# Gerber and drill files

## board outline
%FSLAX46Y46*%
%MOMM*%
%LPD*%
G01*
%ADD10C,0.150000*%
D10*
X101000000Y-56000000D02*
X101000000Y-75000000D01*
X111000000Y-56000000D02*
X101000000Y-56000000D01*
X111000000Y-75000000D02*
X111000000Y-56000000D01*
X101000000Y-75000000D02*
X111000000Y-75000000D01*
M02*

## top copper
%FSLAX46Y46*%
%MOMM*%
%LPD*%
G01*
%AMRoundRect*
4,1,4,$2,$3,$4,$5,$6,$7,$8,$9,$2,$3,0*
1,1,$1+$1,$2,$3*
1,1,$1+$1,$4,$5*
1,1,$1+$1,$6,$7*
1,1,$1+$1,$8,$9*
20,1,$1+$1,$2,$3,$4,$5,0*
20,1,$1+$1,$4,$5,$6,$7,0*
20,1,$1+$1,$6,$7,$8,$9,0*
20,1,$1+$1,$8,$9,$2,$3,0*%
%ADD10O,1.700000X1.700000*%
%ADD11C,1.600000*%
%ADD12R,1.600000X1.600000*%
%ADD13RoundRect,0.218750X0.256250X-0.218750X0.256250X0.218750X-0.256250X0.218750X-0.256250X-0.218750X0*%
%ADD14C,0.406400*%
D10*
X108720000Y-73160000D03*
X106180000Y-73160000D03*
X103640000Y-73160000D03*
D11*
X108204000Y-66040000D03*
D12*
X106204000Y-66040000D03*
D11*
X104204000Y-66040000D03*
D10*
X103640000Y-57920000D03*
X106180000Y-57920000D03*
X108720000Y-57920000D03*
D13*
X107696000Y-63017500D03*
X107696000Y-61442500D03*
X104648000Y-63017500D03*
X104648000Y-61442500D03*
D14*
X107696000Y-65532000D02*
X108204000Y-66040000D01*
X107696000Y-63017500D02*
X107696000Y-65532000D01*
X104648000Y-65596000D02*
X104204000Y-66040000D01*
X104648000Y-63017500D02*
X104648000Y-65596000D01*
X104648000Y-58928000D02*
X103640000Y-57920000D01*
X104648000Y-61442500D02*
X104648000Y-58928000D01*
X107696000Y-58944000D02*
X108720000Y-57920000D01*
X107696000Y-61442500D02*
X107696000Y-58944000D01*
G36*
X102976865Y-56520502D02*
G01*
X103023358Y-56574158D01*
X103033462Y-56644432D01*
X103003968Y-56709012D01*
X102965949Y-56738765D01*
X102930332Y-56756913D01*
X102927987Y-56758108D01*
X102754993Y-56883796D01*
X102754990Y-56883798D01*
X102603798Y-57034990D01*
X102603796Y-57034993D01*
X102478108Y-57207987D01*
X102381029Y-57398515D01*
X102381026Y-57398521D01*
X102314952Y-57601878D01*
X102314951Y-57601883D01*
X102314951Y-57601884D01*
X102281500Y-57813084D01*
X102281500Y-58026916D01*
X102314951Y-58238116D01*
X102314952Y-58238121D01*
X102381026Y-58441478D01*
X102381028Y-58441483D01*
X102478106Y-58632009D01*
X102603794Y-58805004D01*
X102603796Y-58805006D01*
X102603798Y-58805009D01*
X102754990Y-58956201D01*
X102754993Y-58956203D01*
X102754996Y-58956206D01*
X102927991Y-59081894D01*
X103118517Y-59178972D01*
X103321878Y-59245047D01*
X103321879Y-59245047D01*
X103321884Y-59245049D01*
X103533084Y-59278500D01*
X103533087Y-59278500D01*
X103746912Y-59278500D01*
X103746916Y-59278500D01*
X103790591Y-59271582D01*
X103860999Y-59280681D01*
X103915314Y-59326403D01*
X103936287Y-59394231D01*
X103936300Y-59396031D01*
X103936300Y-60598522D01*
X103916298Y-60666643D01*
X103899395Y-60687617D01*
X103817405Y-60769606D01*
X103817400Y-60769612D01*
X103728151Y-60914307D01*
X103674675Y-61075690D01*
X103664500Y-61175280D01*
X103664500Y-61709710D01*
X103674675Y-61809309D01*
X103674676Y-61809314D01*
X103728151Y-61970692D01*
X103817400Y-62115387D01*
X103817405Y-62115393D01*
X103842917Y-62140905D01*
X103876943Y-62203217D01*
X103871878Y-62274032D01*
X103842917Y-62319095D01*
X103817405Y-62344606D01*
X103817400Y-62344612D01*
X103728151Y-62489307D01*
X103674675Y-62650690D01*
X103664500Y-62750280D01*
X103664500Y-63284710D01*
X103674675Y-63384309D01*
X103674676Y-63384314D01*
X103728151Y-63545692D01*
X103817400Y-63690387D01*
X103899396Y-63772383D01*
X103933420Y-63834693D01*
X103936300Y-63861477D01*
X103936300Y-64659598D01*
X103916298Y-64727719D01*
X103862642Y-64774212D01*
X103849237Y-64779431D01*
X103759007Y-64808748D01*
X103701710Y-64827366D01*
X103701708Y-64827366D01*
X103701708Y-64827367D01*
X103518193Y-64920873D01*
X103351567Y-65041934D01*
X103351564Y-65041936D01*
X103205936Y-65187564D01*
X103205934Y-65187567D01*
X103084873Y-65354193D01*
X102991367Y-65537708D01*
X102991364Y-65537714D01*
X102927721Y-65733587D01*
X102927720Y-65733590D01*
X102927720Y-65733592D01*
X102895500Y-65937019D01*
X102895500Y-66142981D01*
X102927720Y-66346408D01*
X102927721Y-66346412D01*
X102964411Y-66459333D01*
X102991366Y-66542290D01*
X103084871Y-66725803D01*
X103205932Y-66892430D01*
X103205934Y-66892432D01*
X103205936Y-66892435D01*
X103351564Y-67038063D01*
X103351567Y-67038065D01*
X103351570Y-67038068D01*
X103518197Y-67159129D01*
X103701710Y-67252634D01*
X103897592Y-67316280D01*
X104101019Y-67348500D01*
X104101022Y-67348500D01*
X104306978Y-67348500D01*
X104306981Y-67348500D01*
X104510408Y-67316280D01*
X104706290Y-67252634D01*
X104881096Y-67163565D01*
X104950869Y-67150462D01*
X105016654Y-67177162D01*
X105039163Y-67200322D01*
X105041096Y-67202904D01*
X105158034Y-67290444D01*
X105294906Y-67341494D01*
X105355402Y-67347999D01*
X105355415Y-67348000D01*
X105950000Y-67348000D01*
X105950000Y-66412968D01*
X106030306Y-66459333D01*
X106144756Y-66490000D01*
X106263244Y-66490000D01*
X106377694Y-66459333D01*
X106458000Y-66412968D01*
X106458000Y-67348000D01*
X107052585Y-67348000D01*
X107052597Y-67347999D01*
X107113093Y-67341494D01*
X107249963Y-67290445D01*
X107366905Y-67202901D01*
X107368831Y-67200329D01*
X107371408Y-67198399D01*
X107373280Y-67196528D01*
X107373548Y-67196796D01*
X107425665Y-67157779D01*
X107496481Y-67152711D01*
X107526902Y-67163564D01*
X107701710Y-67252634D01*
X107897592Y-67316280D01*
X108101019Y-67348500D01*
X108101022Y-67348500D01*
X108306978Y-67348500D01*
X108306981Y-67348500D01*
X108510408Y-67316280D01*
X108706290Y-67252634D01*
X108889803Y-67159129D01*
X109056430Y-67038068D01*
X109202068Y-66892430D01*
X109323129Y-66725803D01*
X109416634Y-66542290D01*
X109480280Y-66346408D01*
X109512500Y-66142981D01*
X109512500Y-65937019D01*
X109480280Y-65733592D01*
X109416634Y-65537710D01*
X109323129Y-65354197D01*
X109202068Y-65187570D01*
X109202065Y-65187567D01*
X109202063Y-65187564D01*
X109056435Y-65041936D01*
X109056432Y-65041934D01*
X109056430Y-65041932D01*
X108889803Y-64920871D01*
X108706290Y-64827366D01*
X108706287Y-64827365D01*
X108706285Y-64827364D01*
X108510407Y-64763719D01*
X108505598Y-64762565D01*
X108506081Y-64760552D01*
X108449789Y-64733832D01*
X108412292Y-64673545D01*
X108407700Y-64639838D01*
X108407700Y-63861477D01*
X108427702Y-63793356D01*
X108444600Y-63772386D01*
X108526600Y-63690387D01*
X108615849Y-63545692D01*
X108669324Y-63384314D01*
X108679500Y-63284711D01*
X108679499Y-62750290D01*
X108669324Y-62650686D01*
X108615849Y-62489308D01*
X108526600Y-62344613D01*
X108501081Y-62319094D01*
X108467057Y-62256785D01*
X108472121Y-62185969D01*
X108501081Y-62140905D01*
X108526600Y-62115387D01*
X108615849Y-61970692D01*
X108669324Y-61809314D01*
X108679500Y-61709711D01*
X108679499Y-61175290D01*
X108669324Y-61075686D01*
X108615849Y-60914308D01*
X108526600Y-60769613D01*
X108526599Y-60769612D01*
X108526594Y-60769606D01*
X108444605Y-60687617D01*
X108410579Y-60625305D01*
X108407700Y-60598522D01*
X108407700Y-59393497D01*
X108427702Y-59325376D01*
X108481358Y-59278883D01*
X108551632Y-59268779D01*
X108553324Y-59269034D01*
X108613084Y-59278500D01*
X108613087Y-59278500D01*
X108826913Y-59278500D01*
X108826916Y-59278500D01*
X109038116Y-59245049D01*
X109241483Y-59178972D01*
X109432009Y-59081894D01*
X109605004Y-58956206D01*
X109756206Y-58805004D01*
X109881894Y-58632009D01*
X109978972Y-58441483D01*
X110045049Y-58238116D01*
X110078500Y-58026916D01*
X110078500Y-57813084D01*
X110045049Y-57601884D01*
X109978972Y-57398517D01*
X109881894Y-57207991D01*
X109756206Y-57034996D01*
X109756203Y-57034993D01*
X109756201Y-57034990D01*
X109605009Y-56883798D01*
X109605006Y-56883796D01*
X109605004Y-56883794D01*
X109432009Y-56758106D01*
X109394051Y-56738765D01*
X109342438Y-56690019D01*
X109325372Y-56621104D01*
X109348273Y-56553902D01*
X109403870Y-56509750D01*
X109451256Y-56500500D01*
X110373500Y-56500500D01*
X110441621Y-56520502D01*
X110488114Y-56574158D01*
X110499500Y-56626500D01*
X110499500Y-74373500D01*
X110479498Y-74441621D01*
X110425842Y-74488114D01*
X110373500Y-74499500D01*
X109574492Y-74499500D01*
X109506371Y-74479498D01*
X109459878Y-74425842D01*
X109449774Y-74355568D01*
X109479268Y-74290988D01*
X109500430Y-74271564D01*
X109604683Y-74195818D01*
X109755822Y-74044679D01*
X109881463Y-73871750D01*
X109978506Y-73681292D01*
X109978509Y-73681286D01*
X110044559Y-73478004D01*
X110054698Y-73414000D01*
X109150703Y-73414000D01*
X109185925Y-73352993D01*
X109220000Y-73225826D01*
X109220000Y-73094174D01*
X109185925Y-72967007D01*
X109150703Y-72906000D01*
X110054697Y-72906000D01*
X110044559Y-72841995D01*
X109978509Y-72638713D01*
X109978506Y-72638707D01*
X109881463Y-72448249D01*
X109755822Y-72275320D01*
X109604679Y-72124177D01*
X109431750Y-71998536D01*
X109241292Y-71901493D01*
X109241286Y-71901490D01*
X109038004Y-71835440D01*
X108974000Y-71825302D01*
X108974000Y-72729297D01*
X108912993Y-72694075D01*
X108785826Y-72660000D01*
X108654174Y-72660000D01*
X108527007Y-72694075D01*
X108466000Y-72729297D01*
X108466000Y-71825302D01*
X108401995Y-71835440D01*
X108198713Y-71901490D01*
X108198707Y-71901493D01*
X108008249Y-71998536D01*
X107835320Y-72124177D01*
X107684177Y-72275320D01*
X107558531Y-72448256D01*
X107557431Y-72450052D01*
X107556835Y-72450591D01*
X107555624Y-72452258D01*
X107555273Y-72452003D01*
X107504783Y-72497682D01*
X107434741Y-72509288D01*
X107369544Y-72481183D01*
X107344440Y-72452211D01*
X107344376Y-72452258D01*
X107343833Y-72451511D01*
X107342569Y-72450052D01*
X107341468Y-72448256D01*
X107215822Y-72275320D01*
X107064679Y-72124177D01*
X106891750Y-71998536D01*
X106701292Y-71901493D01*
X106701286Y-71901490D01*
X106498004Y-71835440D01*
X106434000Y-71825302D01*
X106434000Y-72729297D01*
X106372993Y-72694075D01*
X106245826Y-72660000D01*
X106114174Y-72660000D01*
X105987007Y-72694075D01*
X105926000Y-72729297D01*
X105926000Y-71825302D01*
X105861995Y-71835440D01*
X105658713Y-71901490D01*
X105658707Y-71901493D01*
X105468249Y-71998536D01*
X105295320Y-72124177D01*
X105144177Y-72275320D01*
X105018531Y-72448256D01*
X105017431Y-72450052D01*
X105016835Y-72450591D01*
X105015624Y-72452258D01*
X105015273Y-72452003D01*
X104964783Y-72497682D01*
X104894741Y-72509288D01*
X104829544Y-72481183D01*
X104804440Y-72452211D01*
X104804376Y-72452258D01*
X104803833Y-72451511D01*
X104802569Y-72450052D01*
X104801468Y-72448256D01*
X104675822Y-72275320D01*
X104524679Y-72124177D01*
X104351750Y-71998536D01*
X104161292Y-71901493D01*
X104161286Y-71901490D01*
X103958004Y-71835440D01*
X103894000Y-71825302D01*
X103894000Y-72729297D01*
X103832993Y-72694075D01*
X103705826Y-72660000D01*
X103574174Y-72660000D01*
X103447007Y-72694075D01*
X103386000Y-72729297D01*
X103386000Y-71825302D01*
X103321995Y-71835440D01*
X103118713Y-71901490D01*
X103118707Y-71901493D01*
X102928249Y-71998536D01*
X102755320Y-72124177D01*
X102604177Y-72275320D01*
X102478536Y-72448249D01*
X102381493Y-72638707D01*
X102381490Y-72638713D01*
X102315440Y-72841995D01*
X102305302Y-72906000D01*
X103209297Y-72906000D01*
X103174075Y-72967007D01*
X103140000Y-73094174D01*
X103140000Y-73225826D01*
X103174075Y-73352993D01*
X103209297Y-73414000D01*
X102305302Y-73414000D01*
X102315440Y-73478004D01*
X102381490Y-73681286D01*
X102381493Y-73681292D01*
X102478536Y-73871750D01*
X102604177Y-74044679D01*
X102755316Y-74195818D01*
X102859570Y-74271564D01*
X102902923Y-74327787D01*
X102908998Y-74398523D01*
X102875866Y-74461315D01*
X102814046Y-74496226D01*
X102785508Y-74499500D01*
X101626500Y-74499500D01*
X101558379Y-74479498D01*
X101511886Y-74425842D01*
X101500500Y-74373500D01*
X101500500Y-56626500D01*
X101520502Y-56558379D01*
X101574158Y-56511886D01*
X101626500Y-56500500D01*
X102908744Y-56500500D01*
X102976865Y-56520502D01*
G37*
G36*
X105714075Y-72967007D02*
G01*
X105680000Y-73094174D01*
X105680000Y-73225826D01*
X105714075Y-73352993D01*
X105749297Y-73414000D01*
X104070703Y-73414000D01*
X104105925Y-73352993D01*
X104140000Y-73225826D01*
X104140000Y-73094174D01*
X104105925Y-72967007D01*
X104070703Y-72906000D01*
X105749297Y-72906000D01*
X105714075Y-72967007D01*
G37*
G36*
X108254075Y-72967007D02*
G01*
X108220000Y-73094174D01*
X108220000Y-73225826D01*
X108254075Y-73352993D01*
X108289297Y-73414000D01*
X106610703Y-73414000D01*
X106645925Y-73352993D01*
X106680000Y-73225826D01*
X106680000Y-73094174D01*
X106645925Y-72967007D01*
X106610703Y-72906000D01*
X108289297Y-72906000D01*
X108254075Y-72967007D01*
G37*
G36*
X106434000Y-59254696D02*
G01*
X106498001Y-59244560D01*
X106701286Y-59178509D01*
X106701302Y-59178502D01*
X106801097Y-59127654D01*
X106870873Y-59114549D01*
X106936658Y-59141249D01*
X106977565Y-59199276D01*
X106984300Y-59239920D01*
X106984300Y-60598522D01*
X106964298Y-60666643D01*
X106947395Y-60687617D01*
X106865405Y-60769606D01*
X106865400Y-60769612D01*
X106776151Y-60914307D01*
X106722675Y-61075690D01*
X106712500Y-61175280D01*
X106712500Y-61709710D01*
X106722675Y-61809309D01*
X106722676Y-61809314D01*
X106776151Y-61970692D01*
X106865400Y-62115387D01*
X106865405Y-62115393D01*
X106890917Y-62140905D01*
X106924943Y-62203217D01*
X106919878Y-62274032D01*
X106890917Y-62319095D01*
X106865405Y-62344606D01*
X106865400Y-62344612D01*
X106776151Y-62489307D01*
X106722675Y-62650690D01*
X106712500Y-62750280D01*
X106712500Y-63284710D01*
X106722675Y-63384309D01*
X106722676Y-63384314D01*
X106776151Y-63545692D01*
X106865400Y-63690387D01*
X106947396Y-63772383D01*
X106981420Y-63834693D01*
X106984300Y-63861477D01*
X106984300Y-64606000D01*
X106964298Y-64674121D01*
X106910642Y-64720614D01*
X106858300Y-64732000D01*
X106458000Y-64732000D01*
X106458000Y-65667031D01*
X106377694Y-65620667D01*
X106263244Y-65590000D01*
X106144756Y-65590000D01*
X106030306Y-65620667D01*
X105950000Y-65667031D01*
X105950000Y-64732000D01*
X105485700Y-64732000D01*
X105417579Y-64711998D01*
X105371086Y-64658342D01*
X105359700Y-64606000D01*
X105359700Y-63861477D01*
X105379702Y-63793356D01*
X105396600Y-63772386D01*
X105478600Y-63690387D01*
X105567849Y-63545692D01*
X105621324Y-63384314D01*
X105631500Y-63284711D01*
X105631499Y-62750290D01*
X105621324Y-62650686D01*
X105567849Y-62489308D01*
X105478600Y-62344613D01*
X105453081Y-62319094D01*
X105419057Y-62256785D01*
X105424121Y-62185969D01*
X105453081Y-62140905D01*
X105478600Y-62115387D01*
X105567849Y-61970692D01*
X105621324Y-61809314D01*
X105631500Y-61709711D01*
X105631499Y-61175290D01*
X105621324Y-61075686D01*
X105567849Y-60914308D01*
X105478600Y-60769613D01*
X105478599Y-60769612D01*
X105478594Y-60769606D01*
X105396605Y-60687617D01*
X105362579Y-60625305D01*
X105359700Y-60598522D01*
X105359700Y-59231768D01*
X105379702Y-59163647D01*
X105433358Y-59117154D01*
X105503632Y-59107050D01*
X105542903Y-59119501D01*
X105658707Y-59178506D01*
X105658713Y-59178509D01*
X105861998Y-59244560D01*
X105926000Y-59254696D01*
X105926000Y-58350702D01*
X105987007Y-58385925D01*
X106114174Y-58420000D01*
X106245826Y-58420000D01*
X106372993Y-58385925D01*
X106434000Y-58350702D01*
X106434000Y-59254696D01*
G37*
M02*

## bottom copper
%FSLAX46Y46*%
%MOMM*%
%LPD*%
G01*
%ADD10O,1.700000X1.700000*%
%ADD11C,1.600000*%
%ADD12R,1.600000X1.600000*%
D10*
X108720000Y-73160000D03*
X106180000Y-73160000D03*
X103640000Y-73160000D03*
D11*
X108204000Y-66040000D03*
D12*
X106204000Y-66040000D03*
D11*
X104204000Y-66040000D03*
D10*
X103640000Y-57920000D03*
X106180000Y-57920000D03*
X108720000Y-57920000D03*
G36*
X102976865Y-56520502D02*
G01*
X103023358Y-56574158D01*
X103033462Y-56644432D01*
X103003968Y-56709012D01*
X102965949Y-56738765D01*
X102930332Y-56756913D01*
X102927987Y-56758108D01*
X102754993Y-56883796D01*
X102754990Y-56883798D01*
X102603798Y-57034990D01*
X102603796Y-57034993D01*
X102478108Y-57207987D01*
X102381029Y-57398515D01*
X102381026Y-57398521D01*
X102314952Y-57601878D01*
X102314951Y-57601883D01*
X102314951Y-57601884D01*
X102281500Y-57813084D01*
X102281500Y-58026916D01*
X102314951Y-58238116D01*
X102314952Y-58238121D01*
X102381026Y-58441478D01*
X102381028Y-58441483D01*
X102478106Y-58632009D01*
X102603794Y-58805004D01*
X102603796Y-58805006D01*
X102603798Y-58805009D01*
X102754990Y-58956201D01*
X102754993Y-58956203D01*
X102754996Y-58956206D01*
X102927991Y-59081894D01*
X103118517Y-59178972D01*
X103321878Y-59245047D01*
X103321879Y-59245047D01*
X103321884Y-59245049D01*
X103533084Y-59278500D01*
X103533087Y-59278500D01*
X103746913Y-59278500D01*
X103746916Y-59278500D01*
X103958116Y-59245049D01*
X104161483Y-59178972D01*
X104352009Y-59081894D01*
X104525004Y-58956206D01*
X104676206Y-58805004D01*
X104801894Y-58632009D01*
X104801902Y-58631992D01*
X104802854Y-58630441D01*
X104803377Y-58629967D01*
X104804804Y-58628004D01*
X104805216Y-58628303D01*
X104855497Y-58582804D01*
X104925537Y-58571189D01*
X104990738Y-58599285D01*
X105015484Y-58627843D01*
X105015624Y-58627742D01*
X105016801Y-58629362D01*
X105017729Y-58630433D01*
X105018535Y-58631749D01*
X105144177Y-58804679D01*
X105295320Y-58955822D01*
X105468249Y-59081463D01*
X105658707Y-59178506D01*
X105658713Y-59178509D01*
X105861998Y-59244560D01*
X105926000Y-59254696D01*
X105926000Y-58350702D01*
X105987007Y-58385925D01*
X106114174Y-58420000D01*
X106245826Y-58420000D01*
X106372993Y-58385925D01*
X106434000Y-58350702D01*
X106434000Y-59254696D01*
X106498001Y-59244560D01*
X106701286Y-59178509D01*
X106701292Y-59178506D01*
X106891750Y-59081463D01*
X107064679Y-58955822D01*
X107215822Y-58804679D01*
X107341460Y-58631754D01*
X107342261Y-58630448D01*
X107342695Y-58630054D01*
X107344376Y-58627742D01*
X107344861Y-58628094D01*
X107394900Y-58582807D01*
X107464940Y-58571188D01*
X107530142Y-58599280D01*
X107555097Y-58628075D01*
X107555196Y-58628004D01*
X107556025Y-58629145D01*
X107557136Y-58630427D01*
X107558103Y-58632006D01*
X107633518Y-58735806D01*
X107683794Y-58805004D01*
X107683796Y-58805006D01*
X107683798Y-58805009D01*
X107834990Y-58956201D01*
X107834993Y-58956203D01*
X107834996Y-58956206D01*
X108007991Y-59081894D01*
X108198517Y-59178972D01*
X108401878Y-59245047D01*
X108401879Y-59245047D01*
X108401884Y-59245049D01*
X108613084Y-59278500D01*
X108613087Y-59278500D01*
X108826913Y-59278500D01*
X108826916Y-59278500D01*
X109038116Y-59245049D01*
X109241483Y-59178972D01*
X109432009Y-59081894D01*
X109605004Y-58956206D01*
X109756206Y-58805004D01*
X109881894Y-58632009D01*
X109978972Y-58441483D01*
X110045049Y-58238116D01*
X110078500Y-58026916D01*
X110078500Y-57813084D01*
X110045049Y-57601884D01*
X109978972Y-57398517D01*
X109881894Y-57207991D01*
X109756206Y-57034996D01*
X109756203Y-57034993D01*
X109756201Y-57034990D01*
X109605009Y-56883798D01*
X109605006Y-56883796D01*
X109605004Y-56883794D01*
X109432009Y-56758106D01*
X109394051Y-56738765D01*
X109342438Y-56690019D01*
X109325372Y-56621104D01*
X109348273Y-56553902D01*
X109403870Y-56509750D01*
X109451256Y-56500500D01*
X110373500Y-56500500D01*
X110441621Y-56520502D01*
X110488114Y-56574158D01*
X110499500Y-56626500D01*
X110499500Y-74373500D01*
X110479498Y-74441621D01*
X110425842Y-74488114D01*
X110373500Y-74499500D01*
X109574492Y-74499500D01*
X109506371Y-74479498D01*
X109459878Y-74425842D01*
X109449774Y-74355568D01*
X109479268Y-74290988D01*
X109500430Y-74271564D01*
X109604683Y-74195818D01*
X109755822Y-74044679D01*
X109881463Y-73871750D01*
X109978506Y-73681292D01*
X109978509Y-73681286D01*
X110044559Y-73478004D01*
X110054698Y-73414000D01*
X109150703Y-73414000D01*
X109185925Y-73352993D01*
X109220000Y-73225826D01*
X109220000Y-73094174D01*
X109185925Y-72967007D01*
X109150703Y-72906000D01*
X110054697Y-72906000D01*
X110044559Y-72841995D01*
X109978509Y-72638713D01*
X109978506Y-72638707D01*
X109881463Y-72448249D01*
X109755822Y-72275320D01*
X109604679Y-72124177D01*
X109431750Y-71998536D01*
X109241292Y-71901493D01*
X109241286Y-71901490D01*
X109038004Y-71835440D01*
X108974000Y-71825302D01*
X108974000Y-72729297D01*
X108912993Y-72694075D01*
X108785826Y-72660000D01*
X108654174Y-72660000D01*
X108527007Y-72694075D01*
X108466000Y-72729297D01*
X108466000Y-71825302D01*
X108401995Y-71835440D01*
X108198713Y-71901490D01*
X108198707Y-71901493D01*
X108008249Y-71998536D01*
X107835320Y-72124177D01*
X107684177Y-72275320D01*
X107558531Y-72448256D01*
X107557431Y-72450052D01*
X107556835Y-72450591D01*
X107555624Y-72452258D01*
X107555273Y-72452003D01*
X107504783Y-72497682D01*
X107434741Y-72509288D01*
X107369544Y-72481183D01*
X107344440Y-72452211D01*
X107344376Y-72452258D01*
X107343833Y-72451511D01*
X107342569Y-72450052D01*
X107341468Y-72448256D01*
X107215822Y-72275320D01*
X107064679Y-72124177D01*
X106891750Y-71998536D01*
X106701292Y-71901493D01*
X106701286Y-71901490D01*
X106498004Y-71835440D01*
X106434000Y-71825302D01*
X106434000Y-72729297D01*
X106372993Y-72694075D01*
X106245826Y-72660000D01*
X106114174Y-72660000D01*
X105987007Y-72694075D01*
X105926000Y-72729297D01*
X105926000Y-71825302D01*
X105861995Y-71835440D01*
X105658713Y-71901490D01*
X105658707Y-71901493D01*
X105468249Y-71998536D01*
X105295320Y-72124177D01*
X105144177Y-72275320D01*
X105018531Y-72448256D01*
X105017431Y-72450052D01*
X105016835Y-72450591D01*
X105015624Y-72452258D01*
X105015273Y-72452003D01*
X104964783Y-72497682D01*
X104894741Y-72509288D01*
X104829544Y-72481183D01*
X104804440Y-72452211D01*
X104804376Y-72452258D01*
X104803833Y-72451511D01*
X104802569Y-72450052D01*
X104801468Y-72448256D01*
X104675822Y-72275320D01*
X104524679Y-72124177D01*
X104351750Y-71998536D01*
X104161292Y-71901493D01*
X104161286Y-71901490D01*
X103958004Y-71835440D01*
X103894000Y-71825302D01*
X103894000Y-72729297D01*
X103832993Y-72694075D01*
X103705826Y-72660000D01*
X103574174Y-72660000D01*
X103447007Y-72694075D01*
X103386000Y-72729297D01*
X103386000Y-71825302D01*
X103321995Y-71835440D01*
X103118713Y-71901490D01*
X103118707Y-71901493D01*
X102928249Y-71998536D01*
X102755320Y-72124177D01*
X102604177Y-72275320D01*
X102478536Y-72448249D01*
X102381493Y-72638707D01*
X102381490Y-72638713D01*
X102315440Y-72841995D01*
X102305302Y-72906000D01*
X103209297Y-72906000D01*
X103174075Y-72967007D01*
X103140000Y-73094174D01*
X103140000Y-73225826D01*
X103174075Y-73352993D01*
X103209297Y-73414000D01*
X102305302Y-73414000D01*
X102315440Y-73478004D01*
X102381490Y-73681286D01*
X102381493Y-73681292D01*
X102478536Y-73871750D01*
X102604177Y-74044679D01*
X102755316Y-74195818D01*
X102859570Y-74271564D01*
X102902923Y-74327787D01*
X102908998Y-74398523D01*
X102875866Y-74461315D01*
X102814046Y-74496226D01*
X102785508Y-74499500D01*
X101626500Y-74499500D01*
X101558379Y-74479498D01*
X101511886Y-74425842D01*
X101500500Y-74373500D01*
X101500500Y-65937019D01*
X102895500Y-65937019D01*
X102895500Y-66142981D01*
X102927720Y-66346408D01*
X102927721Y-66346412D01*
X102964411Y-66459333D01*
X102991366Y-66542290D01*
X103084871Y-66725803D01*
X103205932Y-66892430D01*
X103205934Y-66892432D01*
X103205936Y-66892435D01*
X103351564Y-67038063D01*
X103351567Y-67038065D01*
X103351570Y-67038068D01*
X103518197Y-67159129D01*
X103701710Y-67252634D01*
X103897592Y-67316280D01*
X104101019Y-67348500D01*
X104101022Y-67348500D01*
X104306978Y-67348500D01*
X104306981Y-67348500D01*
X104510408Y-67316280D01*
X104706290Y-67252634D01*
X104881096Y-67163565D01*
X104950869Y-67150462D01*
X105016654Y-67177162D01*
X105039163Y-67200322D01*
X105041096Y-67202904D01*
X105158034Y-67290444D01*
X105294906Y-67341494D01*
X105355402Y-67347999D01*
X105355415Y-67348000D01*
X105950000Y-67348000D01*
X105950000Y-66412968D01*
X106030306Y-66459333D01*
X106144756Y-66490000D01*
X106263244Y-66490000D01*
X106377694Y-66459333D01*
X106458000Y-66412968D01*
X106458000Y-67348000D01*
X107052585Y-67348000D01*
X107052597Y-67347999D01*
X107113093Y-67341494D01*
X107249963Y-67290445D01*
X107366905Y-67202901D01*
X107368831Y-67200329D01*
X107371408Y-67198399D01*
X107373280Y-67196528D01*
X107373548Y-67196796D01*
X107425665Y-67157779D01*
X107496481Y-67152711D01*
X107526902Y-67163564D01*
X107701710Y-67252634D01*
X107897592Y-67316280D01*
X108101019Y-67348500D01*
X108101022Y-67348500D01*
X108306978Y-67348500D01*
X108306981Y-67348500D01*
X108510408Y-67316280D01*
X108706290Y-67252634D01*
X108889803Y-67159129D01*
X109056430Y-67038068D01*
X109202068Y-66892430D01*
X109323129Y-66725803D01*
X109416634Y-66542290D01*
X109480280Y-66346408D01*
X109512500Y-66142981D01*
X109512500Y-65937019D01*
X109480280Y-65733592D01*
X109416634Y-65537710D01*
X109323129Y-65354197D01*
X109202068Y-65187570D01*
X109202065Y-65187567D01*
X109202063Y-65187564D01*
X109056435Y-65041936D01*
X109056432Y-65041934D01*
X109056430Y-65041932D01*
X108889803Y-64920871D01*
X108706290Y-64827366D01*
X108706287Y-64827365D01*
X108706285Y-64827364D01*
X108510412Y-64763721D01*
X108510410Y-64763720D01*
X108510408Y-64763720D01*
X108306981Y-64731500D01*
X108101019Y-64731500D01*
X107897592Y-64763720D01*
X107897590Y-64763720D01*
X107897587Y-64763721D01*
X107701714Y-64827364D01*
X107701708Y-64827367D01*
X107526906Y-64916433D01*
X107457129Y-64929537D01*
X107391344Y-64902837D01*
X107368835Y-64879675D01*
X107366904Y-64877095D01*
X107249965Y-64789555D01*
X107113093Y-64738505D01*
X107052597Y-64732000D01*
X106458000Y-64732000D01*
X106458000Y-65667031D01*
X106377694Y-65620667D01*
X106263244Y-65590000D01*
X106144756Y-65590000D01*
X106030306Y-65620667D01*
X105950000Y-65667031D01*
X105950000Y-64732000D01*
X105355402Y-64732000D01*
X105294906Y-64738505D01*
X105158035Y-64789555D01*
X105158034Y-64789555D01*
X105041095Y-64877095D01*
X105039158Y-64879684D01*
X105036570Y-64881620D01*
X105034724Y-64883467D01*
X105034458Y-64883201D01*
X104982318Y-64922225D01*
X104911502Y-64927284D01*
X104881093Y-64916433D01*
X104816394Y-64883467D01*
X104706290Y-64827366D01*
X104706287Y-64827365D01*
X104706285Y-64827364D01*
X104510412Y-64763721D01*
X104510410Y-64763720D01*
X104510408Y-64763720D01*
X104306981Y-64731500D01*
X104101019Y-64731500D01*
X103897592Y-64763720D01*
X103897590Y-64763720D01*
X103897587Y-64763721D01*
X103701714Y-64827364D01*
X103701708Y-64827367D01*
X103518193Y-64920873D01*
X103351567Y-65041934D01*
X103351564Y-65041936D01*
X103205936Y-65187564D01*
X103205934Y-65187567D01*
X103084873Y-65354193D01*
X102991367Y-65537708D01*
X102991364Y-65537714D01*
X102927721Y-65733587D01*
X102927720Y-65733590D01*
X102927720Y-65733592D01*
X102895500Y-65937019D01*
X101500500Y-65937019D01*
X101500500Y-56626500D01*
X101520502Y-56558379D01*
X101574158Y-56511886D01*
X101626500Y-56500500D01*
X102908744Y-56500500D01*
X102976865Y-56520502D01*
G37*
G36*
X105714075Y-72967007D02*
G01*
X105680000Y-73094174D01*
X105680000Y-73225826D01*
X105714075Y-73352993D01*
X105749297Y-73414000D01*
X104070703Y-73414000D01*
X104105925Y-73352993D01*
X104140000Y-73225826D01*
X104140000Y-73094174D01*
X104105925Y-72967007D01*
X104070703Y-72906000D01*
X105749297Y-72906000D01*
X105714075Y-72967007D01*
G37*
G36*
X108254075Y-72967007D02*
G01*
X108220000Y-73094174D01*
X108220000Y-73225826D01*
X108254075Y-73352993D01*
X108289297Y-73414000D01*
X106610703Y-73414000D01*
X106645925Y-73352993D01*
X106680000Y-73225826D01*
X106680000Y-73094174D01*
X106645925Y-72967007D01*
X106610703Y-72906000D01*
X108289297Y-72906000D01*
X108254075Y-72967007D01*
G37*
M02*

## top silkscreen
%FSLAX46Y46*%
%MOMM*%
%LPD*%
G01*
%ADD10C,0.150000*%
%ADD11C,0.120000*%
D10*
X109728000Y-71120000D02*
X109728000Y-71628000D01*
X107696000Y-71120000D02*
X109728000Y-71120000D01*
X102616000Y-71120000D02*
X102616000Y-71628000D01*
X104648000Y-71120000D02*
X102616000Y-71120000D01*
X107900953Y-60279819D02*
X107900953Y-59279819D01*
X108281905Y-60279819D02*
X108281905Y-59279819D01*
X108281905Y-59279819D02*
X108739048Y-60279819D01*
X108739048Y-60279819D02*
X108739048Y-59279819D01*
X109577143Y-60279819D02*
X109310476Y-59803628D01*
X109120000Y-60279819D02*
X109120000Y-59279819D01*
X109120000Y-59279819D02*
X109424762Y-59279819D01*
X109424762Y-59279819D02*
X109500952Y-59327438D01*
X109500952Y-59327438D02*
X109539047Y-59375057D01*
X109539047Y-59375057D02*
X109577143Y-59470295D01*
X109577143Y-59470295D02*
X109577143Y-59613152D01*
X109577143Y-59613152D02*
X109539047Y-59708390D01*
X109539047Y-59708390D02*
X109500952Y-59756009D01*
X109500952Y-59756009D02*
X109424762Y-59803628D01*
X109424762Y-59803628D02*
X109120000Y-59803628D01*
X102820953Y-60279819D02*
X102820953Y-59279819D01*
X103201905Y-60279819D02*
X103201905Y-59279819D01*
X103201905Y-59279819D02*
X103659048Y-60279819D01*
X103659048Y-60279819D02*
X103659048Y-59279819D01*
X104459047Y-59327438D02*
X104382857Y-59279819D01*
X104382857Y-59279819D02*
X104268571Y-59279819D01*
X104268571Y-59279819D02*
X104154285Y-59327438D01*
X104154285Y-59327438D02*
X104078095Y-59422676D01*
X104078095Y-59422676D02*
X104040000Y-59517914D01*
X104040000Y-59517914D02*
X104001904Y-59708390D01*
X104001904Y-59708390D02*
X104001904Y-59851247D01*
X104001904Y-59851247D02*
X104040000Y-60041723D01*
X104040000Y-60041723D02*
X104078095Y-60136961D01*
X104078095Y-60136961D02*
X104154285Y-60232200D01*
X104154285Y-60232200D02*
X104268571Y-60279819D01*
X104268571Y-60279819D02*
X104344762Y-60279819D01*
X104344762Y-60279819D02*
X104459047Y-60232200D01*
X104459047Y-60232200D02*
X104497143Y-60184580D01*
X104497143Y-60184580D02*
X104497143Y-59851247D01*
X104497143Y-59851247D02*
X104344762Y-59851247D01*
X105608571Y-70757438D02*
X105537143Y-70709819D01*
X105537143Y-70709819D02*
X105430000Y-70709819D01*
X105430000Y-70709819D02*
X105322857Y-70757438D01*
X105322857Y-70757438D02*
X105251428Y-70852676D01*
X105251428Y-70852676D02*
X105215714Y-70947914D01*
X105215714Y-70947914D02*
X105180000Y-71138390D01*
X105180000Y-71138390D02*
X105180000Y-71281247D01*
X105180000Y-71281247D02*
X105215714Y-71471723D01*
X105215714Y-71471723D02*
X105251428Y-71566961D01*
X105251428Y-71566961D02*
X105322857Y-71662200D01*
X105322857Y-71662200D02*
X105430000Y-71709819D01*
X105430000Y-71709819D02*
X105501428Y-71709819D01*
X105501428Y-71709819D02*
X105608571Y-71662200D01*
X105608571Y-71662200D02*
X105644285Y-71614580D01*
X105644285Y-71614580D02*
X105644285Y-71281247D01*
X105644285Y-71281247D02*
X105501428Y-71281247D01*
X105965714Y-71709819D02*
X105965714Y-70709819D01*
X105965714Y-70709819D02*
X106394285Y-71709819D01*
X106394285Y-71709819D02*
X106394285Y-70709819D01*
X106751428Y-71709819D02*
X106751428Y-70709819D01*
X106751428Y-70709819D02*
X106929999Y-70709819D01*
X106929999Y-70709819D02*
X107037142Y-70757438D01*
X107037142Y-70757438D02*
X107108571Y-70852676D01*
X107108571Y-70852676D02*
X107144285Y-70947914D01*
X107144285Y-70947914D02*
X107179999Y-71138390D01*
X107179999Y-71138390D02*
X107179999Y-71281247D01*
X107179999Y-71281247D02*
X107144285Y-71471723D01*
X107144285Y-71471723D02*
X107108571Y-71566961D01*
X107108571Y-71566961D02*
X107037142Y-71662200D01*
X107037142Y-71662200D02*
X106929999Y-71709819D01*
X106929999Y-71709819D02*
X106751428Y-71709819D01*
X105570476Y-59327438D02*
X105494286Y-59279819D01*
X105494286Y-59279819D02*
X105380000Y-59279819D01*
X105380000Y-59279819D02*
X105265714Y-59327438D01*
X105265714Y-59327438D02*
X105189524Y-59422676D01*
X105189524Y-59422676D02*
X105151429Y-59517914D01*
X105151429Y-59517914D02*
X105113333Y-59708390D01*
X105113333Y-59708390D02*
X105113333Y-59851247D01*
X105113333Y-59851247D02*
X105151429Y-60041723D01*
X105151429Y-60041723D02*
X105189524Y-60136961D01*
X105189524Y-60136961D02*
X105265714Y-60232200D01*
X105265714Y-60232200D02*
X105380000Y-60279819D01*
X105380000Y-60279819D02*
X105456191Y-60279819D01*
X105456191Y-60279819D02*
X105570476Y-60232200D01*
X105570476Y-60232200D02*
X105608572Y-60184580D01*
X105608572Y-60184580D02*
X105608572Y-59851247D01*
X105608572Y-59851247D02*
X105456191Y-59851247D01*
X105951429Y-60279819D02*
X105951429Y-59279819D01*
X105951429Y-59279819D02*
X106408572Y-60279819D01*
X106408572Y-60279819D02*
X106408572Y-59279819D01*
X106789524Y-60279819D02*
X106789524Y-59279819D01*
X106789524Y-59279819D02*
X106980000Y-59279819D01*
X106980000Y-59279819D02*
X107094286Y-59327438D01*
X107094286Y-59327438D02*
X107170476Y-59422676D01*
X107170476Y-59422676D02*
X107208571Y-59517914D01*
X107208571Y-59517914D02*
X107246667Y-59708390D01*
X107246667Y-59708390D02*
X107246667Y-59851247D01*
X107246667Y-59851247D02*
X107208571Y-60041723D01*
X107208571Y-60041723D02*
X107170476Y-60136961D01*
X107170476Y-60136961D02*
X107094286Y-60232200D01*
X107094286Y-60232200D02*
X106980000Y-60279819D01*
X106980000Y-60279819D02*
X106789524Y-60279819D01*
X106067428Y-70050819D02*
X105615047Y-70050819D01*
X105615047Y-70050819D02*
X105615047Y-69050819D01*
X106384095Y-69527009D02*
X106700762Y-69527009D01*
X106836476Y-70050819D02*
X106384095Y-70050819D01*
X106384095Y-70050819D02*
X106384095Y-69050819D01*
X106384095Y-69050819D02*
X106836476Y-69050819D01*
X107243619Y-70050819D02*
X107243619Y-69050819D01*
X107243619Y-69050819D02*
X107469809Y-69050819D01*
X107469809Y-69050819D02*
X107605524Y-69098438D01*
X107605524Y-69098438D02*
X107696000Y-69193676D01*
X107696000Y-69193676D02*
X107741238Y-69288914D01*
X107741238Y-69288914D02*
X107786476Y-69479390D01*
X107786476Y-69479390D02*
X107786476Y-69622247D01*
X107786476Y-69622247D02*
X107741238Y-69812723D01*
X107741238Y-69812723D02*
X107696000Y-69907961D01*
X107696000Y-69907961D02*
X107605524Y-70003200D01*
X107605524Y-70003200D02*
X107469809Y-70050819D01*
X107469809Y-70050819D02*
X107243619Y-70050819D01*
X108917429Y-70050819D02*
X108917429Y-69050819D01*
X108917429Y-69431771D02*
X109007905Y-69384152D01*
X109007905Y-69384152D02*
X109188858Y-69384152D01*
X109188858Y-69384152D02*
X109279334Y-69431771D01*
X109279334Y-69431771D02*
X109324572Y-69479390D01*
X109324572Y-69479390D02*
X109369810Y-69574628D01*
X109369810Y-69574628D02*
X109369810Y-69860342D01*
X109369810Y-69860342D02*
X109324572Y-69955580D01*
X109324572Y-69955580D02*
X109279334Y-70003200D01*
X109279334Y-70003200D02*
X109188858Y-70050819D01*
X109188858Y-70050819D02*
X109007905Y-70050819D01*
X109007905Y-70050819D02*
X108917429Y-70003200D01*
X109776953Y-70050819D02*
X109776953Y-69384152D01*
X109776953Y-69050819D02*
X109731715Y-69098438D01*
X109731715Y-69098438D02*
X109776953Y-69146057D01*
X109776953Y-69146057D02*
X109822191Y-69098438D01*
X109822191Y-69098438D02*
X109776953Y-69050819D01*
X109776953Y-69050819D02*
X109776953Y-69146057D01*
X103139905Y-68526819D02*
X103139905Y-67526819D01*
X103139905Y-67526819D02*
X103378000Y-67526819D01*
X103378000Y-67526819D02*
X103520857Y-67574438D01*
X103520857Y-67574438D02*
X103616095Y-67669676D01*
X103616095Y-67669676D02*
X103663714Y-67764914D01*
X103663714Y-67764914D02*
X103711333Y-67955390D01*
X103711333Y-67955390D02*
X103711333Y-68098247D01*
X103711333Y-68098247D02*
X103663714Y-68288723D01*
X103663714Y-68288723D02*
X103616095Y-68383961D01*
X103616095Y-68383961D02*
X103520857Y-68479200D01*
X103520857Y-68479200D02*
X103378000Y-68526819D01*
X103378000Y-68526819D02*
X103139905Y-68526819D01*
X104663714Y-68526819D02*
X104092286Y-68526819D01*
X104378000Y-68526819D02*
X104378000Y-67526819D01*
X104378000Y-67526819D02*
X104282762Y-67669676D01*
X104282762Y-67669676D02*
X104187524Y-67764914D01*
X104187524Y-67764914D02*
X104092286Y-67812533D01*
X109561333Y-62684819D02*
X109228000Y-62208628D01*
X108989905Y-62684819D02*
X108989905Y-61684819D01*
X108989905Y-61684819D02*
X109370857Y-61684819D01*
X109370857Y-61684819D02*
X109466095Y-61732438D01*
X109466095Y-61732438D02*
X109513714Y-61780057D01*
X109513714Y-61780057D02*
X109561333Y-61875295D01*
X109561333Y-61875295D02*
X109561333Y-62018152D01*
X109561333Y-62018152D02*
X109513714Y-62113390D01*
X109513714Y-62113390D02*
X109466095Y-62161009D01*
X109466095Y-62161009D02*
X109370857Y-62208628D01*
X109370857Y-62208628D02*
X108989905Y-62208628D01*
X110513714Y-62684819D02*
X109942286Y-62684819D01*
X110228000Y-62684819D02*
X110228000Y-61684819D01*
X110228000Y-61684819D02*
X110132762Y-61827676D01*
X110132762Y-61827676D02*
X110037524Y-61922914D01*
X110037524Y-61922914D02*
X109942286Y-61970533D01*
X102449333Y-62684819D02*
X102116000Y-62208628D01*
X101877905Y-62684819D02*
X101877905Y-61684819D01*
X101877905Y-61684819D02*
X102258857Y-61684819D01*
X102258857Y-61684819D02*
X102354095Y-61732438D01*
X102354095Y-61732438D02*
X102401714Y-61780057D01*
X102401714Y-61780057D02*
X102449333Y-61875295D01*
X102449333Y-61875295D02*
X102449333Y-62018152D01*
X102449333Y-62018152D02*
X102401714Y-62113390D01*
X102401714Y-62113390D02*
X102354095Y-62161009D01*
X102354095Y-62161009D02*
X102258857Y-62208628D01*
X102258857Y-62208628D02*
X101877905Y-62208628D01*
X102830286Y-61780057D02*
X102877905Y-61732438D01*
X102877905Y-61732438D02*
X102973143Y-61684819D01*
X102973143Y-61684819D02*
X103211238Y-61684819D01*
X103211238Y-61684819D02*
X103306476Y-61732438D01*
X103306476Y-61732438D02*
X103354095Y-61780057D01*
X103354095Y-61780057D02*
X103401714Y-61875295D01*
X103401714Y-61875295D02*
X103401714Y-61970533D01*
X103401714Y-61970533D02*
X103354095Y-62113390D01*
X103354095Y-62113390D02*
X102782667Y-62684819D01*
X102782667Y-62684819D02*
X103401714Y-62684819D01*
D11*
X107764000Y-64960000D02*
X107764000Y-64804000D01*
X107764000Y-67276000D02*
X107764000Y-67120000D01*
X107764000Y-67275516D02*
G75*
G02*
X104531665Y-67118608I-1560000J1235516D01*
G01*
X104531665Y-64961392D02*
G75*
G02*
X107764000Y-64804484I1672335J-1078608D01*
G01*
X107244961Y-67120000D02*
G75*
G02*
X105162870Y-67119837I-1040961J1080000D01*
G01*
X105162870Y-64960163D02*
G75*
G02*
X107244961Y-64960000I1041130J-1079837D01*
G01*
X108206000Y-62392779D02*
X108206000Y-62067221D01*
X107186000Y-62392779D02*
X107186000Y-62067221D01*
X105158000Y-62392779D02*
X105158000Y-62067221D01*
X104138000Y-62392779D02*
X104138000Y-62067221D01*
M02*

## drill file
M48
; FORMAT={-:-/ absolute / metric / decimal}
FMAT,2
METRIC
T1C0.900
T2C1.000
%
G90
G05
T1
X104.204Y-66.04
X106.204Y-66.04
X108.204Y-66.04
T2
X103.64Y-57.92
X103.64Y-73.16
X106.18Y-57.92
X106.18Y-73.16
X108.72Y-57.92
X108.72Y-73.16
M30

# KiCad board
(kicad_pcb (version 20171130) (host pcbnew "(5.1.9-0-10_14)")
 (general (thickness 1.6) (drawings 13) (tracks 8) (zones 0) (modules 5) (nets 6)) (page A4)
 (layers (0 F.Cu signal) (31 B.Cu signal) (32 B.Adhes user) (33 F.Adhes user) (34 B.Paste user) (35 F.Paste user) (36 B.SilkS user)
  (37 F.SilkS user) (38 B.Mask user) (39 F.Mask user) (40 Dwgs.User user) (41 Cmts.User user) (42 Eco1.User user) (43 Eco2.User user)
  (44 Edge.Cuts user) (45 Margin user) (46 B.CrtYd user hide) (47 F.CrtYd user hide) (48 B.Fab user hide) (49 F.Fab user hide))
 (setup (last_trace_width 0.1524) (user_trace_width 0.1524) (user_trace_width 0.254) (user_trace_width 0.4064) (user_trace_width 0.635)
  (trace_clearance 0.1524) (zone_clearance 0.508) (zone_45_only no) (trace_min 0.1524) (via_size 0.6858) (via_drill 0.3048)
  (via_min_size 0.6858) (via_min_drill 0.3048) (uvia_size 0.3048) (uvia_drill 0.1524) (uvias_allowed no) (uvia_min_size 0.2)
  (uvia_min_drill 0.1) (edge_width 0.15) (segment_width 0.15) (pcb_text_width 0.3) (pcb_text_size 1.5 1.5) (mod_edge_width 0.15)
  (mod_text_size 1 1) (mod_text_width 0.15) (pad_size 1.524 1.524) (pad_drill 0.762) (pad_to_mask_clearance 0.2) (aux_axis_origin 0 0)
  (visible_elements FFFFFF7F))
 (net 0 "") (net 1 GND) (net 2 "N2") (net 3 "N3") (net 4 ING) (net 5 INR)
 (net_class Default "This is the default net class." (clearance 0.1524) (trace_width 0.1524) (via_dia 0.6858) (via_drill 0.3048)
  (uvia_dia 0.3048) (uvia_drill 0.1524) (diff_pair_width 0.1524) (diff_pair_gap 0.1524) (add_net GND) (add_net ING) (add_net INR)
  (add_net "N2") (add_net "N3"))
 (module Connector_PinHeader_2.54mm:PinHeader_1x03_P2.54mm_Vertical (layer B.Cu) (at 103.64 73.16 270)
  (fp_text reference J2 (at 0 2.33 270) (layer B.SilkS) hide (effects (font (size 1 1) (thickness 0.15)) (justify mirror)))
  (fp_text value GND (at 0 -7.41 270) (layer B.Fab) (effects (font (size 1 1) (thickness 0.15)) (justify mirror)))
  (pad 3 thru_hole oval (at 0 -5.08 270) (size 1.7 1.7) (drill 1) (layers *.Cu *.Mask) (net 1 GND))
  (pad 2 thru_hole oval (at 0 -2.54 270) (size 1.7 1.7) (drill 1) (layers *.Cu *.Mask) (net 1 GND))
  (pad 1 thru_hole oval (at 0 0 270) (size 1.7 1.7) (drill 1) (layers *.Cu *.Mask) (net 1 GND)))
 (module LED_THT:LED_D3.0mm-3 (layer F.Cu) (at 108.704 66.04 180)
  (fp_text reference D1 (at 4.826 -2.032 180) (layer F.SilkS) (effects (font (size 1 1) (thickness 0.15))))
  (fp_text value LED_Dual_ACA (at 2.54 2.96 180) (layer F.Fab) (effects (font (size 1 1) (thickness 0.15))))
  (fp_line (start 0.94 1.08) (end 0.94 1.236) (layer F.SilkS) (width 0.12))
  (fp_line (start 0.94 -1.236) (end 0.94 -1.08) (layer F.SilkS) (width 0.12))
  (fp_arc (start 2.5 0) (end 0.94 -1.235516) (angle 108.8) (layer F.SilkS) (width 0.12))
  (fp_arc (start 2.5 0) (end 0.94 1.235516) (angle -108.8) (layer F.SilkS) (width 0.12))
  (fp_arc (start 2.5 0) (end 1.459039 -1.08) (angle 87.9) (layer F.SilkS) (width 0.12))
  (fp_arc (start 2.5 0) (end 1.459039 1.08) (angle -87.9) (layer F.SilkS) (width 0.12))
  (pad 1 thru_hole circle (at 0.5 0 180) (size 1.6 1.6) (drill 0.9) (layers *.Cu *.Mask) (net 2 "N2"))
  (pad 2 thru_hole rect (at 2.5 0 180) (size 1.6 1.6) (drill 0.9) (layers *.Cu *.Mask) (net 1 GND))
  (pad 3 thru_hole circle (at 4.5 0 180) (size 1.6 1.6) (drill 0.9) (layers *.Cu *.Mask) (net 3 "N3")))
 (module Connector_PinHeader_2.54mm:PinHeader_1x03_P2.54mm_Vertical (layer B.Cu) (at 103.64 57.92 270)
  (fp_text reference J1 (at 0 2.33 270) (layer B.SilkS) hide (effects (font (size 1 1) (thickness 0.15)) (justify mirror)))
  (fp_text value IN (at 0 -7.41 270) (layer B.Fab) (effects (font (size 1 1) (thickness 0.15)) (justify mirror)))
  (pad 1 thru_hole oval (at 0 0 270) (size 1.7 1.7) (drill 1) (layers *.Cu *.Mask) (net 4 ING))
  (pad 2 thru_hole oval (at 0 -2.54 270) (size 1.7 1.7) (drill 1) (layers *.Cu *.Mask) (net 1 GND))
  (pad 3 thru_hole oval (at 0 -5.08 270) (size 1.7 1.7) (drill 1) (layers *.Cu *.Mask) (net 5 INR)))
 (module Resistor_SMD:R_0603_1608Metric (layer F.Cu) (at 107.696 62.23 90)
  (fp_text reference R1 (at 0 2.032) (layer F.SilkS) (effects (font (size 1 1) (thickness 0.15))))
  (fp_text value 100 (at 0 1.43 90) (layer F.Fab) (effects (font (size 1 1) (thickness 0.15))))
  (fp_line (start -0.162779 0.51) (end 0.162779 0.51) (layer F.SilkS) (width 0.12))
  (fp_line (start -0.162779 -0.51) (end 0.162779 -0.51) (layer F.SilkS) (width 0.12))
  (pad 1 smd roundrect (at -0.7875 0 90) (size 0.875 0.95) (layers F.Cu F.Paste F.Mask) (roundrect_rratio 0.25) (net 2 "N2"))
  (pad 2 smd roundrect (at 0.7875 0 90) (size 0.875 0.95) (layers F.Cu F.Paste F.Mask) (roundrect_rratio 0.25) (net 5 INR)))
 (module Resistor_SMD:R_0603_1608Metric (layer F.Cu) (at 104.648 62.23 90)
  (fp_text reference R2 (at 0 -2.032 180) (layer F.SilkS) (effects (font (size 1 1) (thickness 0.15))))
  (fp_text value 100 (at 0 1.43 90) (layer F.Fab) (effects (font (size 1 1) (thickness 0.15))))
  (fp_line (start -0.162779 0.51) (end 0.162779 0.51) (layer F.SilkS) (width 0.12))
  (fp_line (start -0.162779 -0.51) (end 0.162779 -0.51) (layer F.SilkS) (width 0.12))
  (pad 1 smd roundrect (at -0.7875 0 90) (size 0.875 0.95) (layers F.Cu F.Paste F.Mask) (roundrect_rratio 0.25) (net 3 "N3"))
  (pad 2 smd roundrect (at 0.7875 0 90) (size 0.875 0.95) (layers F.Cu F.Paste F.Mask) (roundrect_rratio 0.25) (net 4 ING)))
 (gr_line (start 109.728 71.12) (end 109.728 71.628) (layer F.SilkS) (width 0.15))
 (gr_line (start 107.696 71.12) (end 109.728 71.12) (layer F.SilkS) (width 0.15))
 (gr_line (start 102.616 71.12) (end 102.616 71.628) (layer F.SilkS) (width 0.15))
 (gr_line (start 104.648 71.12) (end 102.616 71.12) (layer F.SilkS) (width 0.15))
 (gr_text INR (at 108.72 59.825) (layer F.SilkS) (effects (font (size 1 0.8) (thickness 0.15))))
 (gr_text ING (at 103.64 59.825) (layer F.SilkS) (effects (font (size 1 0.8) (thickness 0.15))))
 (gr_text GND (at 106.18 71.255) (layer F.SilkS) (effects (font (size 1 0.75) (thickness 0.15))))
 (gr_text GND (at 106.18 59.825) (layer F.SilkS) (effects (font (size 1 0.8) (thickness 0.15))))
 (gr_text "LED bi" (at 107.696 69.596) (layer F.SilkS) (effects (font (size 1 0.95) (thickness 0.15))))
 (gr_line (start 101 56) (end 101 75) (layer Edge.Cuts) (width 0.15))
 (gr_line (start 111 56) (end 101 56) (layer Edge.Cuts) (width 0.15))
 (gr_line (start 111 75) (end 111 56) (layer Edge.Cuts) (width 0.15))
 (gr_line (start 101 75) (end 111 75) (layer Edge.Cuts) (width 0.15))
 (segment (start 107.696 65.532) (end 108.204 66.04) (width 0.4064) (layer F.Cu) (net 2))
 (segment (start 107.696 63.0175) (end 107.696 65.532) (width 0.4064) (layer F.Cu) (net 2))
 (segment (start 104.648 65.596) (end 104.204 66.04) (width 0.4064) (layer F.Cu) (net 3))
 (segment (start 104.648 63.0175) (end 104.648 65.596) (width 0.4064) (layer F.Cu) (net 3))
 (segment (start 104.648 58.928) (end 103.64 57.92) (width 0.4064) (layer F.Cu) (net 4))
 (segment (start 104.648 61.4425) (end 104.648 58.928) (width 0.4064) (layer F.Cu) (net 4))
 (segment (start 107.696 58.944) (end 108.72 57.92) (width 0.4064) (layer F.Cu) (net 5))
 (segment (start 107.696 61.4425) (end 107.696 58.944) (width 0.4064) (layer F.Cu) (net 5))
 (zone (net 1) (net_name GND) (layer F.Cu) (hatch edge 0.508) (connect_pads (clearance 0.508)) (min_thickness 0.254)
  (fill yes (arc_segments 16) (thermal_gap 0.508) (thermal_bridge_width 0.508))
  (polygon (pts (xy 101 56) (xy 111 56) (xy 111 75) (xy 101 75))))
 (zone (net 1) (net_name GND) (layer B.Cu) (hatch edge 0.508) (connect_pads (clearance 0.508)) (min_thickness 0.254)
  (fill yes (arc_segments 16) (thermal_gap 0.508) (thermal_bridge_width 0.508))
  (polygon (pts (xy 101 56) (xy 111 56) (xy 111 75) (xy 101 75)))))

